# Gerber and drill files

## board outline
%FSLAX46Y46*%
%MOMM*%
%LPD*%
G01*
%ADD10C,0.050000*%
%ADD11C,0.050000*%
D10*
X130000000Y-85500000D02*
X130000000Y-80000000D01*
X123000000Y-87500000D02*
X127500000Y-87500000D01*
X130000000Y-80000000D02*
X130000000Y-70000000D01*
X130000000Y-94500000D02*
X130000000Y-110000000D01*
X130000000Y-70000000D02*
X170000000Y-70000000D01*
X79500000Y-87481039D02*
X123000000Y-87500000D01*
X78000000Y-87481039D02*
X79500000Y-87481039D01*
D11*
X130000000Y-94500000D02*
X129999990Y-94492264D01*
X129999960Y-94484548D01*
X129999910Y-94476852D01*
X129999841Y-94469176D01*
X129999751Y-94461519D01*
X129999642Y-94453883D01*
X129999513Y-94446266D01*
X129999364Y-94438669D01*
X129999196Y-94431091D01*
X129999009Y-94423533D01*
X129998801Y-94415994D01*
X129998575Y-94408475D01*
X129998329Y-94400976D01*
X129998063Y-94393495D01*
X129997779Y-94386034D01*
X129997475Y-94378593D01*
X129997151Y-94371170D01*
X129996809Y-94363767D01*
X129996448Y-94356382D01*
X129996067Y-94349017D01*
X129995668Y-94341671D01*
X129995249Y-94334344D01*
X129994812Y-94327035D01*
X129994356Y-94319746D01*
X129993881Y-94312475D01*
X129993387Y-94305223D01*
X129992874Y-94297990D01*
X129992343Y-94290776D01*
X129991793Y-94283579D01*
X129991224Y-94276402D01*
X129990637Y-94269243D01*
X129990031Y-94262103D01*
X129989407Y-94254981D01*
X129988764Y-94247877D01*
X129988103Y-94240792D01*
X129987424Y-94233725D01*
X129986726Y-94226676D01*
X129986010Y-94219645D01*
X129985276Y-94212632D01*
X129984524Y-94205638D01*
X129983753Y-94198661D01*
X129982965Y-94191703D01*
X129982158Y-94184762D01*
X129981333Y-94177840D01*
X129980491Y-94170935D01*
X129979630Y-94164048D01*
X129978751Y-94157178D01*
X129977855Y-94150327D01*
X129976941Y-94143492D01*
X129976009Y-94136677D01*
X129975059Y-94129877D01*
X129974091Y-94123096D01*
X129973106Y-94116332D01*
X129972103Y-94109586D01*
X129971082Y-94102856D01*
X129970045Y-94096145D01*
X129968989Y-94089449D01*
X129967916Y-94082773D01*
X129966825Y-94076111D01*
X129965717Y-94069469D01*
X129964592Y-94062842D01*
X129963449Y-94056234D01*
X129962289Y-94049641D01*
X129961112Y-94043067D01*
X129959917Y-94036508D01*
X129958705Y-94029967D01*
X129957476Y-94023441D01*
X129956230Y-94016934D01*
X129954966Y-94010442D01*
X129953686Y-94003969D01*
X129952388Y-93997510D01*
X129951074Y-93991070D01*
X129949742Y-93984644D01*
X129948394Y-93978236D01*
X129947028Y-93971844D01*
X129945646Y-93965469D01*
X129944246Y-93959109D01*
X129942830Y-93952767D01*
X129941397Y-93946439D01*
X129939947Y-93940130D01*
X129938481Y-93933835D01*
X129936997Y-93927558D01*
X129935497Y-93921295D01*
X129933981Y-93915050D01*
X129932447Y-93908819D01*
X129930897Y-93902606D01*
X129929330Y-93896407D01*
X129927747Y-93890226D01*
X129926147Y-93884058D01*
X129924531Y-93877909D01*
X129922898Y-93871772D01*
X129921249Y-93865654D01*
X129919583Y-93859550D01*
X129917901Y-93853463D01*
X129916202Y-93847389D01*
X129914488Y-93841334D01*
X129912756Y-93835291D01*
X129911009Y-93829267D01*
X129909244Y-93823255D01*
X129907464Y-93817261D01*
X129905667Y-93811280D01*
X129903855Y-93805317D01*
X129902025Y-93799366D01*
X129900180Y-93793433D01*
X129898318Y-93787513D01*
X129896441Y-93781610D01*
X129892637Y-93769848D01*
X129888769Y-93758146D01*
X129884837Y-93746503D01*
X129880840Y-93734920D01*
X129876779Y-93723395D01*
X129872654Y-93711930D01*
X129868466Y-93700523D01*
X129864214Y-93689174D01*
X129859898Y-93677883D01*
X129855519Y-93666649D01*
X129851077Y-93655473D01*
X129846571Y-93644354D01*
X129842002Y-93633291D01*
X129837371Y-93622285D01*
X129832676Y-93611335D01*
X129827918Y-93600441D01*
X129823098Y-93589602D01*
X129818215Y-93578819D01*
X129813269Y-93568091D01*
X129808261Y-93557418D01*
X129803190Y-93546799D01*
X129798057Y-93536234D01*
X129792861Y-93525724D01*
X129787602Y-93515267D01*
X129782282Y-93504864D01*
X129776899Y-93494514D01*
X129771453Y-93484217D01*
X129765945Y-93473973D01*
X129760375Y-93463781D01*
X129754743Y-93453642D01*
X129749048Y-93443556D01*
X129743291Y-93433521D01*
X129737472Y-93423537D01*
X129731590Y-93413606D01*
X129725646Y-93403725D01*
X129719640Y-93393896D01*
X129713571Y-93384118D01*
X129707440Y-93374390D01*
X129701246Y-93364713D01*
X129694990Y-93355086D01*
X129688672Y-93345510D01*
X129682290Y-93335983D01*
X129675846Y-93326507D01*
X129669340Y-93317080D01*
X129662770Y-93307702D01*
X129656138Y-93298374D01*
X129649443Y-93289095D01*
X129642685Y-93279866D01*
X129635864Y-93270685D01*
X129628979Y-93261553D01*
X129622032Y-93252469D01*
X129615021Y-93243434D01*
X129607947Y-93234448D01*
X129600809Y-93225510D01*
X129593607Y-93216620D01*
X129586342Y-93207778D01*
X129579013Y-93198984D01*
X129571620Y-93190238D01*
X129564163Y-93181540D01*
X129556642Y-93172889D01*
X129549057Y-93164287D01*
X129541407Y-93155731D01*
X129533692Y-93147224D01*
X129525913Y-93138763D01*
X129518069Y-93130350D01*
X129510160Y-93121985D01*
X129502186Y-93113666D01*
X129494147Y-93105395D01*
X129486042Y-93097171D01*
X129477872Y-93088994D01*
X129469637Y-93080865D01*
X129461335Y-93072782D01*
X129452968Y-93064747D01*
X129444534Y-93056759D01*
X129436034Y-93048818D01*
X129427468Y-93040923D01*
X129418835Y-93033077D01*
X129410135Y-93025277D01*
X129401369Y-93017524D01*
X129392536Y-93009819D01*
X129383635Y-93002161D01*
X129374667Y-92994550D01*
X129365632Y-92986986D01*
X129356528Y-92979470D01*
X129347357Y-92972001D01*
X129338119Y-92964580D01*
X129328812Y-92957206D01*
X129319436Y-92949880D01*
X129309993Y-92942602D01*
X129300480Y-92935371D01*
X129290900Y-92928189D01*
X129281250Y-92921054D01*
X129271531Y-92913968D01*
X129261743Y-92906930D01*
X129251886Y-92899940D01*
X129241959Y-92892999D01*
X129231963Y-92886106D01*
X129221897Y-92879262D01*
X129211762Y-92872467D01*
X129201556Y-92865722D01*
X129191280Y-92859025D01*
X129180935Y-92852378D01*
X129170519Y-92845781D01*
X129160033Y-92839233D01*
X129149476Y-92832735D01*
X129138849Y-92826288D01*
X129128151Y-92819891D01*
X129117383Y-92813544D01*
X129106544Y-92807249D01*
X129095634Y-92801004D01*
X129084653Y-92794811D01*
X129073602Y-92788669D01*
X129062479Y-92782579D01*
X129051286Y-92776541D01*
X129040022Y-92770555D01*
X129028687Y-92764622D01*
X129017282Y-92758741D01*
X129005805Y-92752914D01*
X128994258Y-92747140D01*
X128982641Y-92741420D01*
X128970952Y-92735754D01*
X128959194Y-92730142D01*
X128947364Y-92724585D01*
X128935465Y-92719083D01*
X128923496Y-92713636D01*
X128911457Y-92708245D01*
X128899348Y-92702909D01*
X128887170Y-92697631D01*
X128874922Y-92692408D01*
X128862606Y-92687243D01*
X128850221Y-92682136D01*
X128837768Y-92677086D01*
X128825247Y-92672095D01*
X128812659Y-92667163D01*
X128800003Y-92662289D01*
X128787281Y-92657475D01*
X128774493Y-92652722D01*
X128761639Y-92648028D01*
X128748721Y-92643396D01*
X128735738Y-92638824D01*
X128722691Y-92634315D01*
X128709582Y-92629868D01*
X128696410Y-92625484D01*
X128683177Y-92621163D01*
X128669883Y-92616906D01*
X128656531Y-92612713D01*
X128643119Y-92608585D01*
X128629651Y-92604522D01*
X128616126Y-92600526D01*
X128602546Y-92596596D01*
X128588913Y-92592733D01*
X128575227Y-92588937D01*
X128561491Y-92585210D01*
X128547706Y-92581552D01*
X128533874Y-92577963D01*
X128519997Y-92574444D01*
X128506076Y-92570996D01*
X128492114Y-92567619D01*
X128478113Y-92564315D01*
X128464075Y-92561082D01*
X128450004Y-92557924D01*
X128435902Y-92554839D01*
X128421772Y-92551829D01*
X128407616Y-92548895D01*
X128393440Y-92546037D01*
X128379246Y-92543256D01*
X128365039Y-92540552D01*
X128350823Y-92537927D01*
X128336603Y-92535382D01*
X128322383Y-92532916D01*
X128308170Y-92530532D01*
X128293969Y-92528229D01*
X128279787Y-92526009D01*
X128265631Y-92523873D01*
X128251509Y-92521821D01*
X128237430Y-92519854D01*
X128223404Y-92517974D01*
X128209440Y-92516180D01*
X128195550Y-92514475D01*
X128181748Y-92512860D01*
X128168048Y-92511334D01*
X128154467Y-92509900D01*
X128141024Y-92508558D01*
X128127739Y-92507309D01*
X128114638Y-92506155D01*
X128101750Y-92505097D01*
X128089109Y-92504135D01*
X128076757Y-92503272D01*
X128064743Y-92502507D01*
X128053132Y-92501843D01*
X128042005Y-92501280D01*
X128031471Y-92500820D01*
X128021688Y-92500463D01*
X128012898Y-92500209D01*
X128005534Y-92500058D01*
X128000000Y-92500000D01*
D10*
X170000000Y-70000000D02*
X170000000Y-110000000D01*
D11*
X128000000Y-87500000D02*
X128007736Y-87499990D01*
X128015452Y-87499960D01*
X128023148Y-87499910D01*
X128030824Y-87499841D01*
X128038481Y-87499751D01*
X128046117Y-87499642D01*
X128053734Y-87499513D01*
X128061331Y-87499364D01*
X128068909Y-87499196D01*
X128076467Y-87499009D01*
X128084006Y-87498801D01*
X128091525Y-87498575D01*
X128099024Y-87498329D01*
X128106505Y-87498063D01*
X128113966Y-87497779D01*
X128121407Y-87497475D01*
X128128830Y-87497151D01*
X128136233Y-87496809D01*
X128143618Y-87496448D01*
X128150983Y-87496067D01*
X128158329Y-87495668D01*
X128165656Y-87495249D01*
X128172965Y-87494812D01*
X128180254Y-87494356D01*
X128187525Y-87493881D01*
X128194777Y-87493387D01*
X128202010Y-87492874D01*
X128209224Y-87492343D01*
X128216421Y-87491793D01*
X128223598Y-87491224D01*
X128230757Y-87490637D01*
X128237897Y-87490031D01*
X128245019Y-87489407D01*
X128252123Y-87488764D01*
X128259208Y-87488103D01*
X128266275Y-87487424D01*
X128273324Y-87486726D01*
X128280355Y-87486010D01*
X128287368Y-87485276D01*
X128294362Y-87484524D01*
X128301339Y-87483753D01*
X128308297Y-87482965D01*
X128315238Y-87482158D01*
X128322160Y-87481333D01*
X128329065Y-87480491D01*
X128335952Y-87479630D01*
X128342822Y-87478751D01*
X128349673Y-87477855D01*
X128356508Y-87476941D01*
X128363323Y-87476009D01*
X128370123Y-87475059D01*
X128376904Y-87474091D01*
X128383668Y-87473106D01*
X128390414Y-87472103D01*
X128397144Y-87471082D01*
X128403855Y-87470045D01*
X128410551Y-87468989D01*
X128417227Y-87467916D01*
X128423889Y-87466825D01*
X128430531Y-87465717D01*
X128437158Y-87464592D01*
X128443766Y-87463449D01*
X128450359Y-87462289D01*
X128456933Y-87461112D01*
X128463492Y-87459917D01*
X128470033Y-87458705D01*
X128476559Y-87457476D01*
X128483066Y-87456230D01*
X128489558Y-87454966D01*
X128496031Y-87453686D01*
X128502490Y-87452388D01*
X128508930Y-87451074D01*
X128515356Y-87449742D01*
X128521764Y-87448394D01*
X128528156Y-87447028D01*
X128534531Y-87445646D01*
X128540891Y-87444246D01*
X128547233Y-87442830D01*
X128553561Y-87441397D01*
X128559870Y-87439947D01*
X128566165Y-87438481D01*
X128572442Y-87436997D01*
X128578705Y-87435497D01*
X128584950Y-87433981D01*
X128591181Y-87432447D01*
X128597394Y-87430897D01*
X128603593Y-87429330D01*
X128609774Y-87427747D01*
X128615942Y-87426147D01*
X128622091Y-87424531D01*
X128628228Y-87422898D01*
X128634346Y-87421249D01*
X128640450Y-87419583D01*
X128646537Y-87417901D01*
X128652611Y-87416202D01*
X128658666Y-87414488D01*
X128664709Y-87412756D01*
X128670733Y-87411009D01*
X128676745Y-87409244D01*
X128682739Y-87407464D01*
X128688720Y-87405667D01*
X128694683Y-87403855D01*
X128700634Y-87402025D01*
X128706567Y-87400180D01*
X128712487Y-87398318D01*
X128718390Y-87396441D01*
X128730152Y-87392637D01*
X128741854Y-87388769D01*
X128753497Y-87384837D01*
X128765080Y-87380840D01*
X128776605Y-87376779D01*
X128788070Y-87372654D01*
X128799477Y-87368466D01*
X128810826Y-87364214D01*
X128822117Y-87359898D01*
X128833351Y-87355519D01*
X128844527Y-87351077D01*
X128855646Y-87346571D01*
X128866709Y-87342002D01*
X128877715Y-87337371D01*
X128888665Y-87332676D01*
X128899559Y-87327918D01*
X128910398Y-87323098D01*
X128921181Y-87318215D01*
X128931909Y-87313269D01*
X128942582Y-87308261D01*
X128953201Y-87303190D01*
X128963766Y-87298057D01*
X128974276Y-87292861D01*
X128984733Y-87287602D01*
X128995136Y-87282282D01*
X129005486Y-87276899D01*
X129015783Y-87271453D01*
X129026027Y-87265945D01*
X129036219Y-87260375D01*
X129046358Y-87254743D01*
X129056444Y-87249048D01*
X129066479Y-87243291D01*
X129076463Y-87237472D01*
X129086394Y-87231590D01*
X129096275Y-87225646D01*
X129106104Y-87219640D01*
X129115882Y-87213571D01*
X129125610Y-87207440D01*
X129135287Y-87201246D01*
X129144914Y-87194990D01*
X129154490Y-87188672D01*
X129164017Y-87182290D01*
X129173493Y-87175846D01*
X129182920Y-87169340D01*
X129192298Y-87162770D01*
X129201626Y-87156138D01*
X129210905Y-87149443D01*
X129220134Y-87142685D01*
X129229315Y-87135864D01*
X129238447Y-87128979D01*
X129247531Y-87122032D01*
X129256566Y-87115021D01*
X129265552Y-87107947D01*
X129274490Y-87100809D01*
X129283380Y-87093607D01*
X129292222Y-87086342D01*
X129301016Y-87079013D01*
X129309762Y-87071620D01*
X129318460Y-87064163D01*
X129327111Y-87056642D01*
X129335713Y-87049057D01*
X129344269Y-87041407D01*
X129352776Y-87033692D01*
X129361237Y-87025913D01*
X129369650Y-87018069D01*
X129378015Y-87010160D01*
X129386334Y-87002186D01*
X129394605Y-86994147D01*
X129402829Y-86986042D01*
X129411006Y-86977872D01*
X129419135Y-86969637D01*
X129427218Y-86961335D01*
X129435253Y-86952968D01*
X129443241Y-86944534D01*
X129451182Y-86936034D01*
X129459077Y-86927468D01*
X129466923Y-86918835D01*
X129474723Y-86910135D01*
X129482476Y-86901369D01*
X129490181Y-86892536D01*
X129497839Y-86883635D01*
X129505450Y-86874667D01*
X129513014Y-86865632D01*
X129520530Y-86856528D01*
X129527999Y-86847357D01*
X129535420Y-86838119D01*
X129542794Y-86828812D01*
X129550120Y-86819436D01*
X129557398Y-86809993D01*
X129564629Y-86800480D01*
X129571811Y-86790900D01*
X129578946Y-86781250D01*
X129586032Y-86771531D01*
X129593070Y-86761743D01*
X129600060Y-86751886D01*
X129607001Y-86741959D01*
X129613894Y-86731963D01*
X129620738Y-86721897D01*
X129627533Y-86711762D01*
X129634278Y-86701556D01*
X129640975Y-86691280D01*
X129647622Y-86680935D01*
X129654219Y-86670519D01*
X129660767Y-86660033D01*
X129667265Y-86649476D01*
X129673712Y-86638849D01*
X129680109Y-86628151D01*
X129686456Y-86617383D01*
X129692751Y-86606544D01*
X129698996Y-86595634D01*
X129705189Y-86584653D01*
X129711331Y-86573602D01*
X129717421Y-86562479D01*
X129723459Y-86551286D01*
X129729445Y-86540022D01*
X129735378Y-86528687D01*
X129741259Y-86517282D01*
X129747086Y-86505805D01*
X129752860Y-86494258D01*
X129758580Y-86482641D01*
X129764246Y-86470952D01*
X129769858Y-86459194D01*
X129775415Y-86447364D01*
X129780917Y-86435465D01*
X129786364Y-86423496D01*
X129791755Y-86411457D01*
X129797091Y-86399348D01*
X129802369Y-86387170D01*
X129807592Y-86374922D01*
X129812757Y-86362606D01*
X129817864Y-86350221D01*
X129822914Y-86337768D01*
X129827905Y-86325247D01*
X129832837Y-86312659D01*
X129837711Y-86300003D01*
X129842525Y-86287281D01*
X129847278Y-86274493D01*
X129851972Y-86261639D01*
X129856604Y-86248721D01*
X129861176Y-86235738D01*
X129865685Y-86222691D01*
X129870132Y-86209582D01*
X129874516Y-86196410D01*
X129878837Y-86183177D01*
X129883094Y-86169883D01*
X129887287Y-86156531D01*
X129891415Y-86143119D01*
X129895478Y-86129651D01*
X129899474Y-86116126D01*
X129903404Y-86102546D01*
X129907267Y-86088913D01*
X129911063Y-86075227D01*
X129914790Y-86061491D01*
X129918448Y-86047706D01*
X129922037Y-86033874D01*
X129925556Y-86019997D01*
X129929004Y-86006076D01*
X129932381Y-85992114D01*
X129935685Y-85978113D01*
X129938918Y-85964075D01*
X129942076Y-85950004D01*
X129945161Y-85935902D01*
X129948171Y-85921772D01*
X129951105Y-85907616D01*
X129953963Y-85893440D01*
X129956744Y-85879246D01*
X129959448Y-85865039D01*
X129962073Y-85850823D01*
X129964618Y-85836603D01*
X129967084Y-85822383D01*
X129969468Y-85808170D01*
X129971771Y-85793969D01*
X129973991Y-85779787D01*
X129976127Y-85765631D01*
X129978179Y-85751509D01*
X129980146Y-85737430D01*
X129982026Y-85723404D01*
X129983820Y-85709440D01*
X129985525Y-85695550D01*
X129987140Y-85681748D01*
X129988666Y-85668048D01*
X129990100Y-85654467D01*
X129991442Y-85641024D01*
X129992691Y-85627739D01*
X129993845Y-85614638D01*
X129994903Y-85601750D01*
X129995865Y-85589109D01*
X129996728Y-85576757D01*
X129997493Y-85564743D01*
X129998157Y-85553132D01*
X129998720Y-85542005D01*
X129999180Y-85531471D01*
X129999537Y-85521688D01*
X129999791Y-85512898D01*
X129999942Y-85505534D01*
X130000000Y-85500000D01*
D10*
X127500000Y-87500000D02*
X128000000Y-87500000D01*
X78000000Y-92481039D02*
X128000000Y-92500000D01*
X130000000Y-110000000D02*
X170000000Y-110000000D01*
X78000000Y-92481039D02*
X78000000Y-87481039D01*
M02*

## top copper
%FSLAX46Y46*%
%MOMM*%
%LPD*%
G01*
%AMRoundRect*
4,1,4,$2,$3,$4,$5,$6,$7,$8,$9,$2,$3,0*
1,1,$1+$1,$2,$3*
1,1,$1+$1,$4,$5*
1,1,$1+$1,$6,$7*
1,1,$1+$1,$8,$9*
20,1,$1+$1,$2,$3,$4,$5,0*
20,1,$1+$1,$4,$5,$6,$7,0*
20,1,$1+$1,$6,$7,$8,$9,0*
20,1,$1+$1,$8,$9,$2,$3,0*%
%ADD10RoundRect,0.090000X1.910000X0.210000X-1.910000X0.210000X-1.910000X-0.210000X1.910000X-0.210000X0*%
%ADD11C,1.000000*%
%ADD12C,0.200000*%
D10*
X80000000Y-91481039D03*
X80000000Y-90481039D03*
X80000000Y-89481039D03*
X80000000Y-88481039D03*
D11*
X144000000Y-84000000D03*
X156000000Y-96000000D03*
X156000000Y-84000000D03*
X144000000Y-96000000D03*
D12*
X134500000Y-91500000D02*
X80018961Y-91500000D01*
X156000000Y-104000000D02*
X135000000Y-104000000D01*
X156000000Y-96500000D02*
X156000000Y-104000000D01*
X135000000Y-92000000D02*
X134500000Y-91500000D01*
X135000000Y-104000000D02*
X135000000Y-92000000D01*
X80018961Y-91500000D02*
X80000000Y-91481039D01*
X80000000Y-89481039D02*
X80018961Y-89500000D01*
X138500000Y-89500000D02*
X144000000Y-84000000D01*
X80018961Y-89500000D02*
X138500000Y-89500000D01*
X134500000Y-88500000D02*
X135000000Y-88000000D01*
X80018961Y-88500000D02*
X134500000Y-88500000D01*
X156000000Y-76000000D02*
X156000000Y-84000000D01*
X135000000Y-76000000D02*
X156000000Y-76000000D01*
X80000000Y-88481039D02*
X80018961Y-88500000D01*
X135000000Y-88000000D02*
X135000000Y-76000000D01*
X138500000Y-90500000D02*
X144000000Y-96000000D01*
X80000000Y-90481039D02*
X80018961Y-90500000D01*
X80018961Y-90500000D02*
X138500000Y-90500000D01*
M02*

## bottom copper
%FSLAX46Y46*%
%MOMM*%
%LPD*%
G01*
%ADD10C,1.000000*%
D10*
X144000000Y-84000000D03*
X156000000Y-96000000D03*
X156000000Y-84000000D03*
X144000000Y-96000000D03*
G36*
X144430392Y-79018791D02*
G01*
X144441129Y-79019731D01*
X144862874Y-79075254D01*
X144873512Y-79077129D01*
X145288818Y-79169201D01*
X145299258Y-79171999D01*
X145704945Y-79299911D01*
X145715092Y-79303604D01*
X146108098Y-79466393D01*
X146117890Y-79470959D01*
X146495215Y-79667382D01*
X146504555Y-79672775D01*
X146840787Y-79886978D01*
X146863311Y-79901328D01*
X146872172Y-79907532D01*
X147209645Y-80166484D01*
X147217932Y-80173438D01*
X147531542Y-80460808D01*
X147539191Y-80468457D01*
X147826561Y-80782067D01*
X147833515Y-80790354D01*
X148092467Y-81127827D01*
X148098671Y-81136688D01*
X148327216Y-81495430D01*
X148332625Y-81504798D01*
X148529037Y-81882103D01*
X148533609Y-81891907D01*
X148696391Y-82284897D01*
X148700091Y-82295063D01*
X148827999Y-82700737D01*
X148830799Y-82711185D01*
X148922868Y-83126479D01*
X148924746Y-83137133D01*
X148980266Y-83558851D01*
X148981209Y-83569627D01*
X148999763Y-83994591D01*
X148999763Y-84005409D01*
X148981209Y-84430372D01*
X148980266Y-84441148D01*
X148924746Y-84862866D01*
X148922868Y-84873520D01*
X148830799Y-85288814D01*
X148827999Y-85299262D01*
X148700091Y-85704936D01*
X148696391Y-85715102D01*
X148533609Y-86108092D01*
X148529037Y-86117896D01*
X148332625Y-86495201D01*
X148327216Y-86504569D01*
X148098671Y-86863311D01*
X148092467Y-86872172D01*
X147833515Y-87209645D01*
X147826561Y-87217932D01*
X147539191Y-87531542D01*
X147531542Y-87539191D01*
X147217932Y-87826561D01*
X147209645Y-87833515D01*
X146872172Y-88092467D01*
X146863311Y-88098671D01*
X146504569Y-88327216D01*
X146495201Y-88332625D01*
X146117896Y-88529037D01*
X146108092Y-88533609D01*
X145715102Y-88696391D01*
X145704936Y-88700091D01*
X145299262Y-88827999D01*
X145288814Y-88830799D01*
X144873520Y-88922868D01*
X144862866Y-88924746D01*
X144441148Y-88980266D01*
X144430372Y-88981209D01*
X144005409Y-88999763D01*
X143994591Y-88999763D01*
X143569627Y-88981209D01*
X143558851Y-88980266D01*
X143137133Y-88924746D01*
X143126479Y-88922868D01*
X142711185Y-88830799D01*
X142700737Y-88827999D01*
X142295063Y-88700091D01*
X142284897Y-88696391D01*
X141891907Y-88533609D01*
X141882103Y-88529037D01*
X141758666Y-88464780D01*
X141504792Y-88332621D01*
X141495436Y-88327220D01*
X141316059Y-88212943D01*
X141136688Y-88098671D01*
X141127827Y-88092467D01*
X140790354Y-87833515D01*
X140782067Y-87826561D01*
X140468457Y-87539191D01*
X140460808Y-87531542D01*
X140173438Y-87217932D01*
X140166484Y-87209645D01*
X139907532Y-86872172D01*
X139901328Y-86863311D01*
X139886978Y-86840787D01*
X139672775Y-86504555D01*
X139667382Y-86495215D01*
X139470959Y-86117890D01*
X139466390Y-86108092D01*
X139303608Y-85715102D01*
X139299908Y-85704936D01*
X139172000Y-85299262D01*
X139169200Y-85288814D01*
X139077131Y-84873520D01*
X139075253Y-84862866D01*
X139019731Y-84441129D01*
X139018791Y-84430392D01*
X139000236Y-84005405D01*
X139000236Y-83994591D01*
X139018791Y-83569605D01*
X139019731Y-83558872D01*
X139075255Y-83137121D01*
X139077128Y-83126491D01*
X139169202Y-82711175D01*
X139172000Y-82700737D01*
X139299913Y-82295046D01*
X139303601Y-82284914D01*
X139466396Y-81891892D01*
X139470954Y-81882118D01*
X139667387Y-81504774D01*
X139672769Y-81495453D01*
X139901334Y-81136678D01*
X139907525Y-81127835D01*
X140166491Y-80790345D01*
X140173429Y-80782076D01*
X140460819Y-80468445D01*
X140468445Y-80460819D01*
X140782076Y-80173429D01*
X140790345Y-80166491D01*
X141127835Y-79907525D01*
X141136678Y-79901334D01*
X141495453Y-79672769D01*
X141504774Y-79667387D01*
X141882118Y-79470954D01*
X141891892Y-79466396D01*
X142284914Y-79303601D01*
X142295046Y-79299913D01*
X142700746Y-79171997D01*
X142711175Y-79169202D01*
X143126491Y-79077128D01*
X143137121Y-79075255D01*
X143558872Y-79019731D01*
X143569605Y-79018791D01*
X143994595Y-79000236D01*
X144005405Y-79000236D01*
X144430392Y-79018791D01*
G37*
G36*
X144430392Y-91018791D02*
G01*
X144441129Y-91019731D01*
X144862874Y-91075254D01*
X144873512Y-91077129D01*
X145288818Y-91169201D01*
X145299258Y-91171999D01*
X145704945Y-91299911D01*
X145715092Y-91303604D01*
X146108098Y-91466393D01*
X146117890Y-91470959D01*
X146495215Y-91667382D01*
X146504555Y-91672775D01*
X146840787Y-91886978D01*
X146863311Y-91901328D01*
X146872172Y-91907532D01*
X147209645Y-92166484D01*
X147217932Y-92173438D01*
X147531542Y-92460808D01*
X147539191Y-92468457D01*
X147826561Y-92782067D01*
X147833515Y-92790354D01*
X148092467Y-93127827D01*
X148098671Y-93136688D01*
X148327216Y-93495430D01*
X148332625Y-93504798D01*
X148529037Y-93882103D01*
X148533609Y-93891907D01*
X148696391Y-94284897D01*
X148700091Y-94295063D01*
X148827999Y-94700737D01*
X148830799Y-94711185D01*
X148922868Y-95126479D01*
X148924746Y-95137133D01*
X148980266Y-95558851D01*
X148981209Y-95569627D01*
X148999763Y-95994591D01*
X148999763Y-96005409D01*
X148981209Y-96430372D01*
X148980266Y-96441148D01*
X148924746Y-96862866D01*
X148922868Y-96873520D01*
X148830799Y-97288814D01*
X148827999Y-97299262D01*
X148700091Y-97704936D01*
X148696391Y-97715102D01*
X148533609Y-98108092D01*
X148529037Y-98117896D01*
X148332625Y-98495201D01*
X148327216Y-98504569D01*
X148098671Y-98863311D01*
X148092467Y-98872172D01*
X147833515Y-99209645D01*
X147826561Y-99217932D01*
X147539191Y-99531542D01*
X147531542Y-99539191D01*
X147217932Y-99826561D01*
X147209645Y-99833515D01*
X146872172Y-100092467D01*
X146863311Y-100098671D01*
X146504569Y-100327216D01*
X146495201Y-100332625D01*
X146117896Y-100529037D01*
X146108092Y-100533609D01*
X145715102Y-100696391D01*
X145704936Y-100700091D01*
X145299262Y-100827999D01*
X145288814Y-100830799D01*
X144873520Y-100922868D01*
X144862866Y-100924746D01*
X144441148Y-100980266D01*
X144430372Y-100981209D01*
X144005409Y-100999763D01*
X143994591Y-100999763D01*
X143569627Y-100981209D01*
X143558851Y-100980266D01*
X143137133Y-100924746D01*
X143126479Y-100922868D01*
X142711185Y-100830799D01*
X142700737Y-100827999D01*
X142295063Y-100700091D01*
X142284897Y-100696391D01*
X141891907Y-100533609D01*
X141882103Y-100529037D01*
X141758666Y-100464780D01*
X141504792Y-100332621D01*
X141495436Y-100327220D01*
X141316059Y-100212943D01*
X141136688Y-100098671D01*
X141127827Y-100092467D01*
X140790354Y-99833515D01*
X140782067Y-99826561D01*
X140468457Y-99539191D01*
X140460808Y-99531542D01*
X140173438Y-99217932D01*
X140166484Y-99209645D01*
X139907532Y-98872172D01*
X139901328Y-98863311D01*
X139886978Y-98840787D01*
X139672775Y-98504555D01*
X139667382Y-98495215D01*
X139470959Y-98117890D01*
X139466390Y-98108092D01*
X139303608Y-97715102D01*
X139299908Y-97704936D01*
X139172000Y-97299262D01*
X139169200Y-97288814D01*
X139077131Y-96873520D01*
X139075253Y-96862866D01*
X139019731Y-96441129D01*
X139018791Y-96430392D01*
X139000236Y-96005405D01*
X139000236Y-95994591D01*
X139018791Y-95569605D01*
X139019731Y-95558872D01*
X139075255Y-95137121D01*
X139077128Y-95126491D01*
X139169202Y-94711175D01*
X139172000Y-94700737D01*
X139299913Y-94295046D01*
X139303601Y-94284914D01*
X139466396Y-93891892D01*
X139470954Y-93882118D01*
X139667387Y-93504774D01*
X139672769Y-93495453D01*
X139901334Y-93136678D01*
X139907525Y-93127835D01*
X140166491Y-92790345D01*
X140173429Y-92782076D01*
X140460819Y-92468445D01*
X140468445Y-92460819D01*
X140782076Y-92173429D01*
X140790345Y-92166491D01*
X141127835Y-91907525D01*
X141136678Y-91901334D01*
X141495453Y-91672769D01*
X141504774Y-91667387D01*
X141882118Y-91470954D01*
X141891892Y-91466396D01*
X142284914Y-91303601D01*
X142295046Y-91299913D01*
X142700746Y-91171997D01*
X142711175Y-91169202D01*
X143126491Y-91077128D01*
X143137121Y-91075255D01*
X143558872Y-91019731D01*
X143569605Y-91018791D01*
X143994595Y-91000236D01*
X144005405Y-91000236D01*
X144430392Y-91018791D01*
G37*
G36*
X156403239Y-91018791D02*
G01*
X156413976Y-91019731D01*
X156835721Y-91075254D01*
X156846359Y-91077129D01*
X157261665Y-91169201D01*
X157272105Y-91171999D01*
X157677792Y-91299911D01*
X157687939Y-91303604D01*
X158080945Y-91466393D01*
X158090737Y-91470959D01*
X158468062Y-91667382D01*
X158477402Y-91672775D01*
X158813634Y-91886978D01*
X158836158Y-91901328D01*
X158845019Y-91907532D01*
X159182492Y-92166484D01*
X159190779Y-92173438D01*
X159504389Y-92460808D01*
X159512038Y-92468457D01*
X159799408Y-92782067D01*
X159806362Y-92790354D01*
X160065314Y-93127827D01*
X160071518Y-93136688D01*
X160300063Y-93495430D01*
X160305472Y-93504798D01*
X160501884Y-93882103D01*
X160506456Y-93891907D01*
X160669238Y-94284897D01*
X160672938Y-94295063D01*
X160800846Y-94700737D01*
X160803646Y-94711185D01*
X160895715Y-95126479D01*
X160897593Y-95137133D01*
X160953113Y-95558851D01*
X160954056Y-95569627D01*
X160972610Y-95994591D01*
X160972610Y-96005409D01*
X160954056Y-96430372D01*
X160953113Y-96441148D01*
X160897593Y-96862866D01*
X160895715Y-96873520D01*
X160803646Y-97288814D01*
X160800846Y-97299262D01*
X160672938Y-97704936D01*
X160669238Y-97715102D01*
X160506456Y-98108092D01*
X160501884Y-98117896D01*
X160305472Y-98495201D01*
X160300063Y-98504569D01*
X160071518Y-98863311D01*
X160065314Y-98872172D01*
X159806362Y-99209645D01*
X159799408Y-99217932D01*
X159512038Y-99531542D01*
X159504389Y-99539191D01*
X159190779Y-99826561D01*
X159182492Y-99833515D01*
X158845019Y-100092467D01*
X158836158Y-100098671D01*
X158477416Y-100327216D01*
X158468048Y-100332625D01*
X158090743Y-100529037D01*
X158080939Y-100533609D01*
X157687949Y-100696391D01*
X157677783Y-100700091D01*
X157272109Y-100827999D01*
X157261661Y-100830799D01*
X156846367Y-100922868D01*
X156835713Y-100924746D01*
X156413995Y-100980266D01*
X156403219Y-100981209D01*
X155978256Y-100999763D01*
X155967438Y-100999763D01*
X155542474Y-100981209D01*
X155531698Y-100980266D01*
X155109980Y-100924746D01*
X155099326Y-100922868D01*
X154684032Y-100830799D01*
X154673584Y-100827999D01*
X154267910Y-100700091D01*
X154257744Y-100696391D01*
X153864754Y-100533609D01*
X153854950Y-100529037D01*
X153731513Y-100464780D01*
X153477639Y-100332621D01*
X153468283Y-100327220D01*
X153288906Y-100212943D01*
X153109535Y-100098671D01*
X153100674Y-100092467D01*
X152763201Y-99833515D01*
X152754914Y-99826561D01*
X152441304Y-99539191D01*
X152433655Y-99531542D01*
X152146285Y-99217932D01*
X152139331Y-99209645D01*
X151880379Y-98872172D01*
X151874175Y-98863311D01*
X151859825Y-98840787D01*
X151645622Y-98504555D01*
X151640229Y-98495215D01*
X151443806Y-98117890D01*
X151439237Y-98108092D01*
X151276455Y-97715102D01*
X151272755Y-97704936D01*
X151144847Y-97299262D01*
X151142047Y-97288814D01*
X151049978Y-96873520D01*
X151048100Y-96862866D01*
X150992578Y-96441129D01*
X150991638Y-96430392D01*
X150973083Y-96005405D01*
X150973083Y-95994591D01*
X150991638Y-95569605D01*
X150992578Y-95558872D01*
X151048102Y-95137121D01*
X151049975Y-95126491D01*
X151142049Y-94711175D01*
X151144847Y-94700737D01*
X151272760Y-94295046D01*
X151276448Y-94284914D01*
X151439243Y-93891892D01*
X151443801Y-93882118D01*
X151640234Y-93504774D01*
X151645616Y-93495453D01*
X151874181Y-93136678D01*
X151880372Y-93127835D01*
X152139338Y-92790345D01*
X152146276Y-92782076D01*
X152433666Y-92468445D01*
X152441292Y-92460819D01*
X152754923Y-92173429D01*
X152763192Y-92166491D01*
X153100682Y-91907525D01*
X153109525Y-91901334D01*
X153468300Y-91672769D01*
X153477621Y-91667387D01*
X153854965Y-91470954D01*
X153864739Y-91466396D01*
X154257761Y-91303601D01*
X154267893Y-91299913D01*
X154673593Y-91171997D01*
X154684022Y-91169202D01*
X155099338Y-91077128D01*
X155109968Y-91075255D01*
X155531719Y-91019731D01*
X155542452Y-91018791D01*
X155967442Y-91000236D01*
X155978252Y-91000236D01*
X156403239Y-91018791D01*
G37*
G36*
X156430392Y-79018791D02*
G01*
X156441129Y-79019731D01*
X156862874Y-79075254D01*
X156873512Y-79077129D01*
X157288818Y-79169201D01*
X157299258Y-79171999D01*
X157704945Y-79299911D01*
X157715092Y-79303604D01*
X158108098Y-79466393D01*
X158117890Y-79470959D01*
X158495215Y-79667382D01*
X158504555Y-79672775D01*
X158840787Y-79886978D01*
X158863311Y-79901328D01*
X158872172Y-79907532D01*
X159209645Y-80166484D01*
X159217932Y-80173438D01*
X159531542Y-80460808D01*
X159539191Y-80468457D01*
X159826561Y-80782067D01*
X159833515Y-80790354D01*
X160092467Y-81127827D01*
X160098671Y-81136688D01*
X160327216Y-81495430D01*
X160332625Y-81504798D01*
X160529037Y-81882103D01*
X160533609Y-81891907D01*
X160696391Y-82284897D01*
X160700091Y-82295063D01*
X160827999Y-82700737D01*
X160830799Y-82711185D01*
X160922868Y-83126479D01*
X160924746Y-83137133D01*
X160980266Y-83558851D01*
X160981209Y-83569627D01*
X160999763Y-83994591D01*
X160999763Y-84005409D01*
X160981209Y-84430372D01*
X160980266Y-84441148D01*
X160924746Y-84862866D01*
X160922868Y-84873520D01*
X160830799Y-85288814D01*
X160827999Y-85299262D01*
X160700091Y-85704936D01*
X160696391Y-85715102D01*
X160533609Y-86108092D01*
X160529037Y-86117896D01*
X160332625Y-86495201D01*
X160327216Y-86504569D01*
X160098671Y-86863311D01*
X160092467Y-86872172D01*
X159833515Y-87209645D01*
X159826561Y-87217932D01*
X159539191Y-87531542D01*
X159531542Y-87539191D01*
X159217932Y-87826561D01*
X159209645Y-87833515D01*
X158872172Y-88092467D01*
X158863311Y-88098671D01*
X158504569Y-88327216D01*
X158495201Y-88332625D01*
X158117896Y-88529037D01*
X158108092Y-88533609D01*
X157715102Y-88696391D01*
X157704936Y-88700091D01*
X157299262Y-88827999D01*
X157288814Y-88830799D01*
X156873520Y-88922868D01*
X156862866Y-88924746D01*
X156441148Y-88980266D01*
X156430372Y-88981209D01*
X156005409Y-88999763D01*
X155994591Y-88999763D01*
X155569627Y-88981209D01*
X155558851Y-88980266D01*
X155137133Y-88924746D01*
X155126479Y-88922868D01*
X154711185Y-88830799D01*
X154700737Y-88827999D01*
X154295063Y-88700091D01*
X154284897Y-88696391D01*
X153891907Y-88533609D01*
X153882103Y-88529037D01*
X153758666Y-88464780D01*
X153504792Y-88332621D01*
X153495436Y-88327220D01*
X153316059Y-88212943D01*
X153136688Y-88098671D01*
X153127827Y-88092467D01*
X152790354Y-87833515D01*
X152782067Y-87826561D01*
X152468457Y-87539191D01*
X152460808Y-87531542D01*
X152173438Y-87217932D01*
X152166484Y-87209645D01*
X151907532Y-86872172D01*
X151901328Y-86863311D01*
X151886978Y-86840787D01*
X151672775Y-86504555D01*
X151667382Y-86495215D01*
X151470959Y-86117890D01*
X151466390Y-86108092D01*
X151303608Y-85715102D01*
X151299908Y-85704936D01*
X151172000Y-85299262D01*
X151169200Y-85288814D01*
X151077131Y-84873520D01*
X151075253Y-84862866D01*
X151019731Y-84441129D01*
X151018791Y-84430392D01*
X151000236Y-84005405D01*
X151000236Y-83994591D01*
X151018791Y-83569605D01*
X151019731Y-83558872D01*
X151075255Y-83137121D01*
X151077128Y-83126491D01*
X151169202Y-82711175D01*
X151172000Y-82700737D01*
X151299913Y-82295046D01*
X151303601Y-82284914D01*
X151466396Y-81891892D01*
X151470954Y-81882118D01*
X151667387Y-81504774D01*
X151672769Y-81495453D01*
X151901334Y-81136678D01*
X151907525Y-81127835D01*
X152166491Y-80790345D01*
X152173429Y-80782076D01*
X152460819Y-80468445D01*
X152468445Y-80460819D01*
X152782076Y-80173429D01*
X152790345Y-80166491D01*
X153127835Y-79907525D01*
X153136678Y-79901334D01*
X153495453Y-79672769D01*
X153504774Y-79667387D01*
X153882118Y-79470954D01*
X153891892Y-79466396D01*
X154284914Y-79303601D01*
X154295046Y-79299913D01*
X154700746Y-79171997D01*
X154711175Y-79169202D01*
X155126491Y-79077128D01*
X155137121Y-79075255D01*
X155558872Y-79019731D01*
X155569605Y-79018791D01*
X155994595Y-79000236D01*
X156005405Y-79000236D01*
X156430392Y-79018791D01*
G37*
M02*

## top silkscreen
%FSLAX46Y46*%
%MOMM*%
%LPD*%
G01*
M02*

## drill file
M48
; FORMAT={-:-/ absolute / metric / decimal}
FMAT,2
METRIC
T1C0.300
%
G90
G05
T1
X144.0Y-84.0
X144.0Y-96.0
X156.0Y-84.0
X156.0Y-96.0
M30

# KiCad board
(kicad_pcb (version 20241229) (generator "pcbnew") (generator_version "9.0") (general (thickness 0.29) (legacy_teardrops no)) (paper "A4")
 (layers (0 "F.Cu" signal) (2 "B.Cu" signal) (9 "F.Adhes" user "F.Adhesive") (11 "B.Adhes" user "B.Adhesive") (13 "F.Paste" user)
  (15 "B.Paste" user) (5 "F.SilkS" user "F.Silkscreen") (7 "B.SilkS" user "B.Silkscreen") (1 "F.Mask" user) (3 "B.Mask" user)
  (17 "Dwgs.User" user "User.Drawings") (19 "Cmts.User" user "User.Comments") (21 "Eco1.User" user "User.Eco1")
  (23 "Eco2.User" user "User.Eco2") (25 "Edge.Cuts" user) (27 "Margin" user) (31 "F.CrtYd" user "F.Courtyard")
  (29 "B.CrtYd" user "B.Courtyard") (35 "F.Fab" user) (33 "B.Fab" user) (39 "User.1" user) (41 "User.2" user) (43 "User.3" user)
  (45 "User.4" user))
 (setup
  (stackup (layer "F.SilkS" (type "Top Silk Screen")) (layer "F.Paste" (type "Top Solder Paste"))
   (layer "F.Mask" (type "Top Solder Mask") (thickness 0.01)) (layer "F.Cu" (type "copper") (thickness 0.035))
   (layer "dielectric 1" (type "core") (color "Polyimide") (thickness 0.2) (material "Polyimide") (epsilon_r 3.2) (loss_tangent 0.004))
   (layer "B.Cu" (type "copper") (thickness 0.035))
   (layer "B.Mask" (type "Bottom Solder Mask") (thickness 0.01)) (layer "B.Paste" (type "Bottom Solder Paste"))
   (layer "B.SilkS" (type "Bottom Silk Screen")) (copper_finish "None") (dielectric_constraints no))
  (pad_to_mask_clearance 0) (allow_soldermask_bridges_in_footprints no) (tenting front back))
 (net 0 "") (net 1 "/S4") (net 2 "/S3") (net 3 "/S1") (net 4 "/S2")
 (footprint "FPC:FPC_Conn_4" (layer "F.Cu") (at 80 89.981039 180)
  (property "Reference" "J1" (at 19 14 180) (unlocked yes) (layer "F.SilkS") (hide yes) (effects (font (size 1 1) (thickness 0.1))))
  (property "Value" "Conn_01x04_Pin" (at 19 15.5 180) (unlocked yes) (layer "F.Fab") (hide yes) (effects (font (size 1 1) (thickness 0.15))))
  (fp_line (start 2 -2.5) (end 2 2.5) (stroke (width 0.05) (type solid)) (layer "Edge.Cuts"))
  (pad "1" smd roundrect (at 0 -1.5 180) (size 4 0.6) (layers "F.Cu" "F.Mask") (roundrect_rratio 0.15) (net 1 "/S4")
   (thermal_bridge_angle 45))
  (pad "2" smd roundrect (at 0 -0.5 180) (size 4 0.6) (layers "F.Cu" "F.Mask") (roundrect_rratio 0.15) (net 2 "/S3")
   (thermal_bridge_angle 45))
  (pad "3" smd roundrect (at 0 0.5 180) (size 4 0.6) (layers "F.Cu" "F.Mask") (roundrect_rratio 0.15) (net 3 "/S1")
   (thermal_bridge_angle 45))
  (pad "4" smd roundrect (at 0 1.5 180) (size 4 0.6) (layers "F.Cu" "F.Mask") (roundrect_rratio 0.15) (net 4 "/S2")
   (thermal_bridge_angle 45)))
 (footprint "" (layer "F.Cu") (at 144 84)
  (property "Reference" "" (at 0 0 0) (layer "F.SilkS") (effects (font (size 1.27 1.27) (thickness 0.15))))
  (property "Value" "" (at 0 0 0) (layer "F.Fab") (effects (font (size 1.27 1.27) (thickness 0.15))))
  (pad "1" thru_hole circle (at 0 0) (size 1 1) (drill 0.3) (layers "*.Cu") (remove_unused_layers no) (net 3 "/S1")))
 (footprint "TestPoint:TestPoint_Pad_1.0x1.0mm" (layer "F.Cu") (at 156 96)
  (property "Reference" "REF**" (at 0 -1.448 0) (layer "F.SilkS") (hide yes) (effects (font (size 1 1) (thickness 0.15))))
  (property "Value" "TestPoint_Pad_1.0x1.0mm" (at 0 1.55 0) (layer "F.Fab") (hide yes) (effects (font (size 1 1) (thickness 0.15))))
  (pad "1" thru_hole circle (at 0 0) (size 1 1) (drill 0.3) (layers "*.Cu") (remove_unused_layers no) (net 1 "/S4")))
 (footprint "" (layer "F.Cu") (at 156 84)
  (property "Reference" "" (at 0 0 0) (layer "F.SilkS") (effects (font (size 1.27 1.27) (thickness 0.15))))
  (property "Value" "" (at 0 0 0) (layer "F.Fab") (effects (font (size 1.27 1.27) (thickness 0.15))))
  (pad "1" thru_hole circle (at 0 0) (size 1 1) (drill 0.3) (layers "*.Cu") (remove_unused_layers no) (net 4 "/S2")))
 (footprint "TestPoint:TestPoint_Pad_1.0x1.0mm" (layer "F.Cu") (at 144 96)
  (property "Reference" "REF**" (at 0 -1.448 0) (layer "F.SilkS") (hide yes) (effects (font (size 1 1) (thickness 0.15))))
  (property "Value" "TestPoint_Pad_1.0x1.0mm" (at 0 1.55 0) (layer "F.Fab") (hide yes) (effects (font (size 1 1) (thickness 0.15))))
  (pad "1" thru_hole circle (at 0 0) (size 1 1) (drill 0.3) (layers "*.Cu") (remove_unused_layers no) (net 2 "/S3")))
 (gr_line (start 130 85.5) (end 130 80) (stroke (width 0.05) (type default)) (layer "Edge.Cuts"))
 (gr_line (start 123 87.5) (end 127.5 87.5) (stroke (width 0.05) (type default)) (layer "Edge.Cuts"))
 (gr_line (start 130 80) (end 130 70) (stroke (width 0.05) (type default)) (layer "Edge.Cuts"))
 (gr_line (start 130 94.5) (end 130 110) (stroke (width 0.05) (type default)) (layer "Edge.Cuts"))
 (gr_line (start 130 70) (end 170 70) (stroke (width 0.05) (type default)) (layer "Edge.Cuts"))
 (gr_line (start 79.5 87.481039) (end 123 87.5) (stroke (width 0.05) (type default)) (layer "Edge.Cuts"))
 (gr_line (start 78 87.481039) (end 79.5 87.481039) (stroke (width 0.05) (type default)) (layer "Edge.Cuts"))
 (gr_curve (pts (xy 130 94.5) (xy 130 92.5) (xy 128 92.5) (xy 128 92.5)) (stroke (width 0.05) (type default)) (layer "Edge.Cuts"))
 (gr_line (start 170 70) (end 170 110) (stroke (width 0.05) (type default)) (layer "Edge.Cuts"))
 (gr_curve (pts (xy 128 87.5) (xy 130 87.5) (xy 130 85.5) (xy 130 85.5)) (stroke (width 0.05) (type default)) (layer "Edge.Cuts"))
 (gr_line (start 127.5 87.5) (end 128 87.5) (stroke (width 0.05) (type default)) (layer "Edge.Cuts"))
 (gr_line (start 78 92.481039) (end 128 92.5) (stroke (width 0.05) (type default)) (layer "Edge.Cuts"))
 (gr_line (start 130 110) (end 170 110) (stroke (width 0.05) (type default)) (layer "Edge.Cuts"))
 (segment (start 134.5 91.5) (end 80.018961 91.5) (width 0.2) (layer "F.Cu") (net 1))
 (segment (start 156 104) (end 135 104) (width 0.2) (layer "F.Cu") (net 1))
 (segment (start 156 96.5) (end 156 104) (width 0.2) (layer "F.Cu") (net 1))
 (segment (start 135 92) (end 134.5 91.5) (width 0.2) (layer "F.Cu") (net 1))
 (segment (start 135 104) (end 135 92) (width 0.2) (layer "F.Cu") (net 1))
 (segment (start 80.018961 91.5) (end 80 91.481039) (width 0.2) (layer "F.Cu") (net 1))
 (segment (start 80 89.481039) (end 80.018961 89.5) (width 0.2) (layer "F.Cu") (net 3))
 (segment (start 138.5 89.5) (end 144 84) (width 0.2) (layer "F.Cu") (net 3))
 (segment (start 80.018961 89.5) (end 138.5 89.5) (width 0.2) (layer "F.Cu") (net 3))
 (segment (start 134.5 88.5) (end 135 88) (width 0.2) (layer "F.Cu") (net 4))
 (segment (start 80.018961 88.5) (end 134.5 88.5) (width 0.2) (layer "F.Cu") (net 4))
 (segment (start 156 76) (end 156 84) (width 0.2) (layer "F.Cu") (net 4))
 (segment (start 135 76) (end 156 76) (width 0.2) (layer "F.Cu") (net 4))
 (segment (start 80 88.481039) (end 80.018961 88.5) (width 0.2) (layer "F.Cu") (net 4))
 (segment (start 135 88) (end 135 76) (width 0.2) (layer "F.Cu") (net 4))
 (segment (start 138.5 90.5) (end 144 96) (width 0.2) (layer "F.Cu") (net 2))
 (segment (start 80 90.481039) (end 80.018961 90.5) (width 0.2) (layer "F.Cu") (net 2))
 (segment (start 80.018961 90.5) (end 138.5 90.5) (width 0.2) (layer "F.Cu") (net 2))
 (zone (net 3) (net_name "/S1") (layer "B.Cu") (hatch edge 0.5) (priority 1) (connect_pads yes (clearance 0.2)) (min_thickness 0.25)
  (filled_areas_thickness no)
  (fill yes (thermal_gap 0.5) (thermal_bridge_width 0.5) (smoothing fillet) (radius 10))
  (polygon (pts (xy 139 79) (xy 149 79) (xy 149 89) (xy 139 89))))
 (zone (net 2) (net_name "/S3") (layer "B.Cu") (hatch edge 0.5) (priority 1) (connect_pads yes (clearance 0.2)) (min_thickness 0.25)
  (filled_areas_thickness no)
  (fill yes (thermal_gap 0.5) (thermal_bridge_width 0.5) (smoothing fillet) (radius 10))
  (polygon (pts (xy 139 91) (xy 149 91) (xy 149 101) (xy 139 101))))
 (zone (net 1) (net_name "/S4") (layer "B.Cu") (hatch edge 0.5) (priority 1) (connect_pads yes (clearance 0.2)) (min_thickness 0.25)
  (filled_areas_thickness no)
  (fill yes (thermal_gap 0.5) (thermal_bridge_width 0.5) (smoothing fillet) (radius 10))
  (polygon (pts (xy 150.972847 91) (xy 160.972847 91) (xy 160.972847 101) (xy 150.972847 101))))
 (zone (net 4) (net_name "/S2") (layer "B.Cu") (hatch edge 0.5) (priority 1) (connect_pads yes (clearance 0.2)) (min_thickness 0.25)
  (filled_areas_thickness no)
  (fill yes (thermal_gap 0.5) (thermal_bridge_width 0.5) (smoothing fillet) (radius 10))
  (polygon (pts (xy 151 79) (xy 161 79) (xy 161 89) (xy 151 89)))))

